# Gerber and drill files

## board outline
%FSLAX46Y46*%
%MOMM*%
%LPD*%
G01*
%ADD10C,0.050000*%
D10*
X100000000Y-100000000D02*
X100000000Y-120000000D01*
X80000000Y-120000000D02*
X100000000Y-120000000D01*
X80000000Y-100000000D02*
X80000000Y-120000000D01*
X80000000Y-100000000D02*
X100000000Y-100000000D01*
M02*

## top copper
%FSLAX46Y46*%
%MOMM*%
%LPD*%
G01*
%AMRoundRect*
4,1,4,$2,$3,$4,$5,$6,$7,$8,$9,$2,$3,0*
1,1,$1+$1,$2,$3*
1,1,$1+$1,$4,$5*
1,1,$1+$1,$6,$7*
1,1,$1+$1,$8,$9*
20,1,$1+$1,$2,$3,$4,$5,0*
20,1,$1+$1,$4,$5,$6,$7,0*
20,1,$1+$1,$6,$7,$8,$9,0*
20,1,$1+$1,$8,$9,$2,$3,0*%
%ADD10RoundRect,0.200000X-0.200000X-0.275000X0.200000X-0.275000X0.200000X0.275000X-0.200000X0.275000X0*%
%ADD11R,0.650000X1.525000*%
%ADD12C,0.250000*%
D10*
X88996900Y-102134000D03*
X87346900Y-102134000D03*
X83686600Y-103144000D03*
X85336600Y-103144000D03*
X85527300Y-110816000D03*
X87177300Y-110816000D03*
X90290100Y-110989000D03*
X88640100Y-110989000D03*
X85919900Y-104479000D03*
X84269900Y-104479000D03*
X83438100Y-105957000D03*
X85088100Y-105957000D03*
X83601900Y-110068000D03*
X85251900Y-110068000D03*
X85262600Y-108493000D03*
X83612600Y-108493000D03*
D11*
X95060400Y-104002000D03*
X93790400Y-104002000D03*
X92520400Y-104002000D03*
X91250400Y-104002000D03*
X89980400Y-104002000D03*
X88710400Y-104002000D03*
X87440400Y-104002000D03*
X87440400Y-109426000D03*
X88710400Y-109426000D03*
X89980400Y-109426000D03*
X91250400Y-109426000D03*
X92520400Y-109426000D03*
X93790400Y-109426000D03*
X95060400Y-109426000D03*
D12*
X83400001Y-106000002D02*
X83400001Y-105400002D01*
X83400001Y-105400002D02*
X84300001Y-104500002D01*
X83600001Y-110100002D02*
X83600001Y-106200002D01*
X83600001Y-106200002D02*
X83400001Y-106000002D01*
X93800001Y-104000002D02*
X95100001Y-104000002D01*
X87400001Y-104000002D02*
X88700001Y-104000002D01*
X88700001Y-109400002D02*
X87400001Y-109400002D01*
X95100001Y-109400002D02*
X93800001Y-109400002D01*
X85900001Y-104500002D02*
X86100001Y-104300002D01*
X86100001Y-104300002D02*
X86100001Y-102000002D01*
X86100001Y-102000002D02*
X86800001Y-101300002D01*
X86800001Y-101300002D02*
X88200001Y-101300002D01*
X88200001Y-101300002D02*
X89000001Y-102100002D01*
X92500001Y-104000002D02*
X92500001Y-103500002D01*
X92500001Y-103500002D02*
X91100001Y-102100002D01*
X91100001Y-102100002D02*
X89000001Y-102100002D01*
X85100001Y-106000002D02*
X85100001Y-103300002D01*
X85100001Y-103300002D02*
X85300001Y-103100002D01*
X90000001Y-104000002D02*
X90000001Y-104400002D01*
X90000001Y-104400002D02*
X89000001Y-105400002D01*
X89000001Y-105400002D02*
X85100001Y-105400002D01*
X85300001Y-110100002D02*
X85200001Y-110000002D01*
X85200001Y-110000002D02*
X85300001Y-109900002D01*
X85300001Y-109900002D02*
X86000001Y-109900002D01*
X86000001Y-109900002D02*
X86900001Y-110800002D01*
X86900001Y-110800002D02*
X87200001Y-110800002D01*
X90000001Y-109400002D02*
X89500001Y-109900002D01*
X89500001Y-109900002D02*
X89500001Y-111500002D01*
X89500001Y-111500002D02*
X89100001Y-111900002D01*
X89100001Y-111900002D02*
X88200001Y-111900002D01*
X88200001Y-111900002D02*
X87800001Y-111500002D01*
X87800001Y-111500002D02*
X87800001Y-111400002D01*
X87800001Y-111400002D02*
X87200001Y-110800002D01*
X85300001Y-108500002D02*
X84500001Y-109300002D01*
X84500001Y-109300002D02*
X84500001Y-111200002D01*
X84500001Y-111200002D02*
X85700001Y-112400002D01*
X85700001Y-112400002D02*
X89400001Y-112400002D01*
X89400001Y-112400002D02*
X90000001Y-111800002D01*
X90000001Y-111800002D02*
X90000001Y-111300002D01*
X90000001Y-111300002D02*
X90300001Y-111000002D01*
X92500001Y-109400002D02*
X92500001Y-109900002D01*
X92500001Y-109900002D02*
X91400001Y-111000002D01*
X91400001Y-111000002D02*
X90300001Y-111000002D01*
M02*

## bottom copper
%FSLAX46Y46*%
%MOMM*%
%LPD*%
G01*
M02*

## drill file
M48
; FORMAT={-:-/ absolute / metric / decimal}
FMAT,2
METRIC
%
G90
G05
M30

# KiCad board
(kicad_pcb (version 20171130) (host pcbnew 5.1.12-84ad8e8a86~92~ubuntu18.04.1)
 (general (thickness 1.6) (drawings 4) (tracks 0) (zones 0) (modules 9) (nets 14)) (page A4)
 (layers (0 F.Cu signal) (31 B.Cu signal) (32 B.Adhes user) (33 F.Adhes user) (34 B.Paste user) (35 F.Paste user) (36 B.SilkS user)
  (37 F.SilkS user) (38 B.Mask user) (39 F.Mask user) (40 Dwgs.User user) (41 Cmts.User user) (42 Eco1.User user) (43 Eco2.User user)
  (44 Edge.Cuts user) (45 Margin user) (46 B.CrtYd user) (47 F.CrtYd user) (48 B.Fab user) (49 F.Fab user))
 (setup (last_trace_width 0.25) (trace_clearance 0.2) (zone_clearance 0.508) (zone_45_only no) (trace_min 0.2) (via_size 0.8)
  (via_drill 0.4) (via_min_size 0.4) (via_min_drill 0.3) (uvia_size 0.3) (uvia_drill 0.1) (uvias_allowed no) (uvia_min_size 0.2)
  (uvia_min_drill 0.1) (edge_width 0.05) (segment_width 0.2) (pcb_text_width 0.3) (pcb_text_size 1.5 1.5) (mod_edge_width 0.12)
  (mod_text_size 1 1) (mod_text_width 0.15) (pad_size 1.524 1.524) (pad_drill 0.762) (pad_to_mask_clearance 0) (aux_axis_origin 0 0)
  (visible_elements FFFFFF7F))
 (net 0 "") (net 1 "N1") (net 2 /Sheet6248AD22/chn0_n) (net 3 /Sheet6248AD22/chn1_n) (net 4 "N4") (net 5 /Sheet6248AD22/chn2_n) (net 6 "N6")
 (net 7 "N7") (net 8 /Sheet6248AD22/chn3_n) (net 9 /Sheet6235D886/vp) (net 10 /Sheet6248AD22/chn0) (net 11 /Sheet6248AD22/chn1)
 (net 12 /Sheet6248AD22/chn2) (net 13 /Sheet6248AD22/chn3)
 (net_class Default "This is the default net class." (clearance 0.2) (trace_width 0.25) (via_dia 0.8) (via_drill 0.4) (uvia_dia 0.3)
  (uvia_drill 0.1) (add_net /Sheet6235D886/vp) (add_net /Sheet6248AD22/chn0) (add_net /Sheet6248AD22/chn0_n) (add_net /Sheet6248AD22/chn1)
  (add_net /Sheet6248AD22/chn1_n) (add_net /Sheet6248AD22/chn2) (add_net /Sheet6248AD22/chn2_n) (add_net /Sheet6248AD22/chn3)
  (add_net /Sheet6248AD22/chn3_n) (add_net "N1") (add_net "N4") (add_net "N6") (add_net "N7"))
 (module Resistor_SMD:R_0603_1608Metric (layer F.Cu) (at 88.171900 102.134000)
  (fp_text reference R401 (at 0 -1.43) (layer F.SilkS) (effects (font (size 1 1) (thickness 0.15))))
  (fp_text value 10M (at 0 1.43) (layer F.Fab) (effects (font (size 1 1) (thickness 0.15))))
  (pad 2 smd roundrect (at 0.825 0) (size 0.8 0.95) (layers F.Cu F.Mask F.Paste) (roundrect_rratio 0.25) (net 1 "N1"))
  (pad 1 smd roundrect (at -0.825 0) (size 0.8 0.95) (layers F.Cu F.Mask F.Paste) (roundrect_rratio 0.25) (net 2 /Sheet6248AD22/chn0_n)))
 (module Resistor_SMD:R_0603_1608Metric (layer F.Cu) (at 84.511600 103.144000)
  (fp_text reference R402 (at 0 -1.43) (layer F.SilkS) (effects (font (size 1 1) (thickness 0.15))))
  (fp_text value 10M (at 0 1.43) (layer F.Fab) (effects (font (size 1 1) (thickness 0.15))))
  (pad 1 smd roundrect (at -0.825 0) (size 0.8 0.95) (layers F.Cu F.Mask F.Paste) (roundrect_rratio 0.25) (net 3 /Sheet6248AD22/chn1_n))
  (pad 2 smd roundrect (at 0.825 0) (size 0.8 0.95) (layers F.Cu F.Mask F.Paste) (roundrect_rratio 0.25) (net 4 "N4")))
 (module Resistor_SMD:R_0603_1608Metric (layer F.Cu) (at 86.352300 110.816000)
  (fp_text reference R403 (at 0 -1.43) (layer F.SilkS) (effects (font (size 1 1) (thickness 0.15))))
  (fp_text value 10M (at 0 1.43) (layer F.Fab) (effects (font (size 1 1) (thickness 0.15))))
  (pad 1 smd roundrect (at -0.825 0) (size 0.8 0.95) (layers F.Cu F.Mask F.Paste) (roundrect_rratio 0.25) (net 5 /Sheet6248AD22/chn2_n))
  (pad 2 smd roundrect (at 0.825 0) (size 0.8 0.95) (layers F.Cu F.Mask F.Paste) (roundrect_rratio 0.25) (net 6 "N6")))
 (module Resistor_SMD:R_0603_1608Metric (layer F.Cu) (at 89.465100 110.989000)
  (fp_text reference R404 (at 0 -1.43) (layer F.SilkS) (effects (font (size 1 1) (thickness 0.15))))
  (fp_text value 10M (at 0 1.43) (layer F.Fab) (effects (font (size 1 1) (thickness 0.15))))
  (pad 2 smd roundrect (at 0.825 0) (size 0.8 0.95) (layers F.Cu F.Mask F.Paste) (roundrect_rratio 0.25) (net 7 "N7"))
  (pad 1 smd roundrect (at -0.825 0) (size 0.8 0.95) (layers F.Cu F.Mask F.Paste) (roundrect_rratio 0.25) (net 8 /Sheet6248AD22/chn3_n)))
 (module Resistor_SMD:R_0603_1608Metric (layer F.Cu) (at 85.094900 104.479000)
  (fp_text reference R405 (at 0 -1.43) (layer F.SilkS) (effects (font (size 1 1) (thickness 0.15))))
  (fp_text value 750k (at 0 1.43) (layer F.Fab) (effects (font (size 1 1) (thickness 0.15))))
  (pad 2 smd roundrect (at 0.825 0) (size 0.8 0.95) (layers F.Cu F.Mask F.Paste) (roundrect_rratio 0.25) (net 1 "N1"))
  (pad 1 smd roundrect (at -0.825 0) (size 0.8 0.95) (layers F.Cu F.Mask F.Paste) (roundrect_rratio 0.25) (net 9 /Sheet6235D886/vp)))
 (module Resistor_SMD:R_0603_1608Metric (layer F.Cu) (at 84.263100 105.957000)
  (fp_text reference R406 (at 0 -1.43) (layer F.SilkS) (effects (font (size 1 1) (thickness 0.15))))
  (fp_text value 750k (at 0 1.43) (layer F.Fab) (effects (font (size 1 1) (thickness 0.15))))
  (pad 1 smd roundrect (at -0.825 0) (size 0.8 0.95) (layers F.Cu F.Mask F.Paste) (roundrect_rratio 0.25) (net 9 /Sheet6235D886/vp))
  (pad 2 smd roundrect (at 0.825 0) (size 0.8 0.95) (layers F.Cu F.Mask F.Paste) (roundrect_rratio 0.25) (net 4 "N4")))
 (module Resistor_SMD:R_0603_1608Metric (layer F.Cu) (at 84.426900 110.068000)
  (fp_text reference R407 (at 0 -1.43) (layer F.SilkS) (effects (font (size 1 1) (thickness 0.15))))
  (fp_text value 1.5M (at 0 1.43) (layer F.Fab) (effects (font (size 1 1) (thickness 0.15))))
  (pad 1 smd roundrect (at -0.825 0) (size 0.8 0.95) (layers F.Cu F.Mask F.Paste) (roundrect_rratio 0.25) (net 9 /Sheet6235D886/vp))
  (pad 2 smd roundrect (at 0.825 0) (size 0.8 0.95) (layers F.Cu F.Mask F.Paste) (roundrect_rratio 0.25) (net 6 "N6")))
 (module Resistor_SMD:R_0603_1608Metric (layer F.Cu) (at 84.437600 108.493000)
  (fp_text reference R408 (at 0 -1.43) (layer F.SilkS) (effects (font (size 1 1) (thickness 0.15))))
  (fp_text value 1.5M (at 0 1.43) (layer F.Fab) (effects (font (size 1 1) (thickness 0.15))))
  (pad 2 smd roundrect (at 0.825 0) (size 0.8 0.95) (layers F.Cu F.Mask F.Paste) (roundrect_rratio 0.25) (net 7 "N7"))
  (pad 1 smd roundrect (at -0.825 0) (size 0.8 0.95) (layers F.Cu F.Mask F.Paste) (roundrect_rratio 0.25) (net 9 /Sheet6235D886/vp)))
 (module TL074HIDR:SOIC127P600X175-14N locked (layer F.Cu) (at 91.250400 106.714000 270.000000)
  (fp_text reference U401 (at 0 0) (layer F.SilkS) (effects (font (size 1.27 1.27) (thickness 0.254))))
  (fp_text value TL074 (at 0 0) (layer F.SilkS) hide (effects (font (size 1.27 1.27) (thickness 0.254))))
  (pad 1 smd rect (at -2.712 -3.81) (size 0.65 1.525) (layers F.Cu F.Mask F.Paste) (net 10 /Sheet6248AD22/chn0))
  (pad 2 smd rect (at -2.712 -2.54) (size 0.65 1.525) (layers F.Cu F.Mask F.Paste) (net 10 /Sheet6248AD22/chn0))
  (pad 3 smd rect (at -2.712 -1.27) (size 0.65 1.525) (layers F.Cu F.Mask F.Paste) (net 1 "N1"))
  (pad 4 smd rect (at -2.712 0) (size 0.65 1.525) (layers F.Cu F.Mask F.Paste))
  (pad 5 smd rect (at -2.712 1.27) (size 0.65 1.525) (layers F.Cu F.Mask F.Paste) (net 4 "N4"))
  (pad 6 smd rect (at -2.712 2.54) (size 0.65 1.525) (layers F.Cu F.Mask F.Paste) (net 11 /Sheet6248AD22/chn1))
  (pad 7 smd rect (at -2.712 3.81) (size 0.65 1.525) (layers F.Cu F.Mask F.Paste) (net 11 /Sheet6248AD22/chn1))
  (pad 8 smd rect (at 2.712 3.81) (size 0.65 1.525) (layers F.Cu F.Mask F.Paste) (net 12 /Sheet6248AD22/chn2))
  (pad 9 smd rect (at 2.712 2.54) (size 0.65 1.525) (layers F.Cu F.Mask F.Paste) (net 12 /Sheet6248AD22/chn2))
  (pad 10 smd rect (at 2.712 1.27) (size 0.65 1.525) (layers F.Cu F.Mask F.Paste) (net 6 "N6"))
  (pad 11 smd rect (at 2.712 0) (size 0.65 1.525) (layers F.Cu F.Mask F.Paste))
  (pad 12 smd rect (at 2.712 -1.27) (size 0.65 1.525) (layers F.Cu F.Mask F.Paste) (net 7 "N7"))
  (pad 13 smd rect (at 2.712 -2.54) (size 0.65 1.525) (layers F.Cu F.Mask F.Paste) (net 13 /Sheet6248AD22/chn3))
  (pad 14 smd rect (at 2.712 -3.81) (size 0.65 1.525) (layers F.Cu F.Mask F.Paste) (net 13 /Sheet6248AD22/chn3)))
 (gr_line (start 100 100) (end 100 120) (layer Edge.Cuts) (width 0.05))
 (gr_line (start 80 120) (end 100 120) (layer Edge.Cuts) (width 0.05))
 (gr_line (start 80 100) (end 80 120) (layer Edge.Cuts) (width 0.05))
 (gr_line (start 80 100) (end 100 100) (layer Edge.Cuts) (width 0.05))
 (segment (start 83.400001 106.000002) (end 83.400001 105.400002) (width 0.250000) (layer F.Cu) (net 9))
 (segment (start 83.400001 105.400002) (end 84.300001 104.500002) (width 0.250000) (layer F.Cu) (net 9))
 (segment (start 83.600001 110.100002) (end 83.600001 106.200002) (width 0.250000) (layer F.Cu) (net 9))
 (segment (start 83.600001 106.200002) (end 83.400001 106.000002) (width 0.250000) (layer F.Cu) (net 9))
 (segment (start 93.800001 104.000002) (end 95.100001 104.000002) (width 0.250000) (layer F.Cu) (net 10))
 (segment (start 87.400001 104.000002) (end 88.700001 104.000002) (width 0.250000) (layer F.Cu) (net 11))
 (segment (start 88.700001 109.400002) (end 87.400001 109.400002) (width 0.250000) (layer F.Cu) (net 12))
 (segment (start 95.100001 109.400002) (end 93.800001 109.400002) (width 0.250000) (layer F.Cu) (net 13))
 (segment (start 85.900001 104.500002) (end 86.100001 104.300002) (width 0.250000) (layer F.Cu) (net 1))
 (segment (start 86.100001 104.300002) (end 86.100001 102.000002) (width 0.250000) (layer F.Cu) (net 1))
 (segment (start 86.100001 102.000002) (end 86.800001 101.300002) (width 0.250000) (layer F.Cu) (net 1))
 (segment (start 86.800001 101.300002) (end 88.200001 101.300002) (width 0.250000) (layer F.Cu) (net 1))
 (segment (start 88.200001 101.300002) (end 89.000001 102.100002) (width 0.250000) (layer F.Cu) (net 1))
 (segment (start 92.500001 104.000002) (end 92.500001 103.500002) (width 0.250000) (layer F.Cu) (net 1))
 (segment (start 92.500001 103.500002) (end 91.100001 102.100002) (width 0.250000) (layer F.Cu) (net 1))
 (segment (start 91.100001 102.100002) (end 89.000001 102.100002) (width 0.250000) (layer F.Cu) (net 1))
 (segment (start 85.100001 106.000002) (end 85.100001 103.300002) (width 0.250000) (layer F.Cu) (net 4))
 (segment (start 85.100001 103.300002) (end 85.300001 103.100002) (width 0.250000) (layer F.Cu) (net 4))
 (segment (start 90.000001 104.000002) (end 90.000001 104.400002) (width 0.250000) (layer F.Cu) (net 4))
 (segment (start 90.000001 104.400002) (end 89.000001 105.400002) (width 0.250000) (layer F.Cu) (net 4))
 (segment (start 89.000001 105.400002) (end 85.100001 105.400002) (width 0.250000) (layer F.Cu) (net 4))
 (segment (start 85.300001 110.100002) (end 85.200001 110.000002) (width 0.250000) (layer F.Cu) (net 6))
 (segment (start 85.200001 110.000002) (end 85.300001 109.900002) (width 0.250000) (layer F.Cu) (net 6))
 (segment (start 85.300001 109.900002) (end 86.000001 109.900002) (width 0.250000) (layer F.Cu) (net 6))
 (segment (start 86.000001 109.900002) (end 86.900001 110.800002) (width 0.250000) (layer F.Cu) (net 6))
 (segment (start 86.900001 110.800002) (end 87.200001 110.800002) (width 0.250000) (layer F.Cu) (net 6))
 (segment (start 90.000001 109.400002) (end 89.500001 109.900002) (width 0.250000) (layer F.Cu) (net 6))
 (segment (start 89.500001 109.900002) (end 89.500001 111.500002) (width 0.250000) (layer F.Cu) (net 6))
 (segment (start 89.500001 111.500002) (end 89.100001 111.900002) (width 0.250000) (layer F.Cu) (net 6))
 (segment (start 89.100001 111.900002) (end 88.200001 111.900002) (width 0.250000) (layer F.Cu) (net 6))
 (segment (start 88.200001 111.900002) (end 87.800001 111.500002) (width 0.250000) (layer F.Cu) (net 6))
 (segment (start 87.800001 111.500002) (end 87.800001 111.400002) (width 0.250000) (layer F.Cu) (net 6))
 (segment (start 87.800001 111.400002) (end 87.200001 110.800002) (width 0.250000) (layer F.Cu) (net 6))
 (segment (start 85.300001 108.500002) (end 84.500001 109.300002) (width 0.250000) (layer F.Cu) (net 7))
 (segment (start 84.500001 109.300002) (end 84.500001 111.200002) (width 0.250000) (layer F.Cu) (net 7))
 (segment (start 84.500001 111.200002) (end 85.700001 112.400002) (width 0.250000) (layer F.Cu) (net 7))
 (segment (start 85.700001 112.400002) (end 89.400001 112.400002) (width 0.250000) (layer F.Cu) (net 7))
 (segment (start 89.400001 112.400002) (end 90.000001 111.800002) (width 0.250000) (layer F.Cu) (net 7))
 (segment (start 90.000001 111.800002) (end 90.000001 111.300002) (width 0.250000) (layer F.Cu) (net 7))
 (segment (start 90.000001 111.300002) (end 90.300001 111.000002) (width 0.250000) (layer F.Cu) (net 7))
 (segment (start 92.500001 109.400002) (end 92.500001 109.900002) (width 0.250000) (layer F.Cu) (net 7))
 (segment (start 92.500001 109.900002) (end 91.400001 111.000002) (width 0.250000) (layer F.Cu) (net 7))
 (segment (start 91.400001 111.000002) (end 90.300001 111.000002) (width 0.250000) (layer F.Cu) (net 7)))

